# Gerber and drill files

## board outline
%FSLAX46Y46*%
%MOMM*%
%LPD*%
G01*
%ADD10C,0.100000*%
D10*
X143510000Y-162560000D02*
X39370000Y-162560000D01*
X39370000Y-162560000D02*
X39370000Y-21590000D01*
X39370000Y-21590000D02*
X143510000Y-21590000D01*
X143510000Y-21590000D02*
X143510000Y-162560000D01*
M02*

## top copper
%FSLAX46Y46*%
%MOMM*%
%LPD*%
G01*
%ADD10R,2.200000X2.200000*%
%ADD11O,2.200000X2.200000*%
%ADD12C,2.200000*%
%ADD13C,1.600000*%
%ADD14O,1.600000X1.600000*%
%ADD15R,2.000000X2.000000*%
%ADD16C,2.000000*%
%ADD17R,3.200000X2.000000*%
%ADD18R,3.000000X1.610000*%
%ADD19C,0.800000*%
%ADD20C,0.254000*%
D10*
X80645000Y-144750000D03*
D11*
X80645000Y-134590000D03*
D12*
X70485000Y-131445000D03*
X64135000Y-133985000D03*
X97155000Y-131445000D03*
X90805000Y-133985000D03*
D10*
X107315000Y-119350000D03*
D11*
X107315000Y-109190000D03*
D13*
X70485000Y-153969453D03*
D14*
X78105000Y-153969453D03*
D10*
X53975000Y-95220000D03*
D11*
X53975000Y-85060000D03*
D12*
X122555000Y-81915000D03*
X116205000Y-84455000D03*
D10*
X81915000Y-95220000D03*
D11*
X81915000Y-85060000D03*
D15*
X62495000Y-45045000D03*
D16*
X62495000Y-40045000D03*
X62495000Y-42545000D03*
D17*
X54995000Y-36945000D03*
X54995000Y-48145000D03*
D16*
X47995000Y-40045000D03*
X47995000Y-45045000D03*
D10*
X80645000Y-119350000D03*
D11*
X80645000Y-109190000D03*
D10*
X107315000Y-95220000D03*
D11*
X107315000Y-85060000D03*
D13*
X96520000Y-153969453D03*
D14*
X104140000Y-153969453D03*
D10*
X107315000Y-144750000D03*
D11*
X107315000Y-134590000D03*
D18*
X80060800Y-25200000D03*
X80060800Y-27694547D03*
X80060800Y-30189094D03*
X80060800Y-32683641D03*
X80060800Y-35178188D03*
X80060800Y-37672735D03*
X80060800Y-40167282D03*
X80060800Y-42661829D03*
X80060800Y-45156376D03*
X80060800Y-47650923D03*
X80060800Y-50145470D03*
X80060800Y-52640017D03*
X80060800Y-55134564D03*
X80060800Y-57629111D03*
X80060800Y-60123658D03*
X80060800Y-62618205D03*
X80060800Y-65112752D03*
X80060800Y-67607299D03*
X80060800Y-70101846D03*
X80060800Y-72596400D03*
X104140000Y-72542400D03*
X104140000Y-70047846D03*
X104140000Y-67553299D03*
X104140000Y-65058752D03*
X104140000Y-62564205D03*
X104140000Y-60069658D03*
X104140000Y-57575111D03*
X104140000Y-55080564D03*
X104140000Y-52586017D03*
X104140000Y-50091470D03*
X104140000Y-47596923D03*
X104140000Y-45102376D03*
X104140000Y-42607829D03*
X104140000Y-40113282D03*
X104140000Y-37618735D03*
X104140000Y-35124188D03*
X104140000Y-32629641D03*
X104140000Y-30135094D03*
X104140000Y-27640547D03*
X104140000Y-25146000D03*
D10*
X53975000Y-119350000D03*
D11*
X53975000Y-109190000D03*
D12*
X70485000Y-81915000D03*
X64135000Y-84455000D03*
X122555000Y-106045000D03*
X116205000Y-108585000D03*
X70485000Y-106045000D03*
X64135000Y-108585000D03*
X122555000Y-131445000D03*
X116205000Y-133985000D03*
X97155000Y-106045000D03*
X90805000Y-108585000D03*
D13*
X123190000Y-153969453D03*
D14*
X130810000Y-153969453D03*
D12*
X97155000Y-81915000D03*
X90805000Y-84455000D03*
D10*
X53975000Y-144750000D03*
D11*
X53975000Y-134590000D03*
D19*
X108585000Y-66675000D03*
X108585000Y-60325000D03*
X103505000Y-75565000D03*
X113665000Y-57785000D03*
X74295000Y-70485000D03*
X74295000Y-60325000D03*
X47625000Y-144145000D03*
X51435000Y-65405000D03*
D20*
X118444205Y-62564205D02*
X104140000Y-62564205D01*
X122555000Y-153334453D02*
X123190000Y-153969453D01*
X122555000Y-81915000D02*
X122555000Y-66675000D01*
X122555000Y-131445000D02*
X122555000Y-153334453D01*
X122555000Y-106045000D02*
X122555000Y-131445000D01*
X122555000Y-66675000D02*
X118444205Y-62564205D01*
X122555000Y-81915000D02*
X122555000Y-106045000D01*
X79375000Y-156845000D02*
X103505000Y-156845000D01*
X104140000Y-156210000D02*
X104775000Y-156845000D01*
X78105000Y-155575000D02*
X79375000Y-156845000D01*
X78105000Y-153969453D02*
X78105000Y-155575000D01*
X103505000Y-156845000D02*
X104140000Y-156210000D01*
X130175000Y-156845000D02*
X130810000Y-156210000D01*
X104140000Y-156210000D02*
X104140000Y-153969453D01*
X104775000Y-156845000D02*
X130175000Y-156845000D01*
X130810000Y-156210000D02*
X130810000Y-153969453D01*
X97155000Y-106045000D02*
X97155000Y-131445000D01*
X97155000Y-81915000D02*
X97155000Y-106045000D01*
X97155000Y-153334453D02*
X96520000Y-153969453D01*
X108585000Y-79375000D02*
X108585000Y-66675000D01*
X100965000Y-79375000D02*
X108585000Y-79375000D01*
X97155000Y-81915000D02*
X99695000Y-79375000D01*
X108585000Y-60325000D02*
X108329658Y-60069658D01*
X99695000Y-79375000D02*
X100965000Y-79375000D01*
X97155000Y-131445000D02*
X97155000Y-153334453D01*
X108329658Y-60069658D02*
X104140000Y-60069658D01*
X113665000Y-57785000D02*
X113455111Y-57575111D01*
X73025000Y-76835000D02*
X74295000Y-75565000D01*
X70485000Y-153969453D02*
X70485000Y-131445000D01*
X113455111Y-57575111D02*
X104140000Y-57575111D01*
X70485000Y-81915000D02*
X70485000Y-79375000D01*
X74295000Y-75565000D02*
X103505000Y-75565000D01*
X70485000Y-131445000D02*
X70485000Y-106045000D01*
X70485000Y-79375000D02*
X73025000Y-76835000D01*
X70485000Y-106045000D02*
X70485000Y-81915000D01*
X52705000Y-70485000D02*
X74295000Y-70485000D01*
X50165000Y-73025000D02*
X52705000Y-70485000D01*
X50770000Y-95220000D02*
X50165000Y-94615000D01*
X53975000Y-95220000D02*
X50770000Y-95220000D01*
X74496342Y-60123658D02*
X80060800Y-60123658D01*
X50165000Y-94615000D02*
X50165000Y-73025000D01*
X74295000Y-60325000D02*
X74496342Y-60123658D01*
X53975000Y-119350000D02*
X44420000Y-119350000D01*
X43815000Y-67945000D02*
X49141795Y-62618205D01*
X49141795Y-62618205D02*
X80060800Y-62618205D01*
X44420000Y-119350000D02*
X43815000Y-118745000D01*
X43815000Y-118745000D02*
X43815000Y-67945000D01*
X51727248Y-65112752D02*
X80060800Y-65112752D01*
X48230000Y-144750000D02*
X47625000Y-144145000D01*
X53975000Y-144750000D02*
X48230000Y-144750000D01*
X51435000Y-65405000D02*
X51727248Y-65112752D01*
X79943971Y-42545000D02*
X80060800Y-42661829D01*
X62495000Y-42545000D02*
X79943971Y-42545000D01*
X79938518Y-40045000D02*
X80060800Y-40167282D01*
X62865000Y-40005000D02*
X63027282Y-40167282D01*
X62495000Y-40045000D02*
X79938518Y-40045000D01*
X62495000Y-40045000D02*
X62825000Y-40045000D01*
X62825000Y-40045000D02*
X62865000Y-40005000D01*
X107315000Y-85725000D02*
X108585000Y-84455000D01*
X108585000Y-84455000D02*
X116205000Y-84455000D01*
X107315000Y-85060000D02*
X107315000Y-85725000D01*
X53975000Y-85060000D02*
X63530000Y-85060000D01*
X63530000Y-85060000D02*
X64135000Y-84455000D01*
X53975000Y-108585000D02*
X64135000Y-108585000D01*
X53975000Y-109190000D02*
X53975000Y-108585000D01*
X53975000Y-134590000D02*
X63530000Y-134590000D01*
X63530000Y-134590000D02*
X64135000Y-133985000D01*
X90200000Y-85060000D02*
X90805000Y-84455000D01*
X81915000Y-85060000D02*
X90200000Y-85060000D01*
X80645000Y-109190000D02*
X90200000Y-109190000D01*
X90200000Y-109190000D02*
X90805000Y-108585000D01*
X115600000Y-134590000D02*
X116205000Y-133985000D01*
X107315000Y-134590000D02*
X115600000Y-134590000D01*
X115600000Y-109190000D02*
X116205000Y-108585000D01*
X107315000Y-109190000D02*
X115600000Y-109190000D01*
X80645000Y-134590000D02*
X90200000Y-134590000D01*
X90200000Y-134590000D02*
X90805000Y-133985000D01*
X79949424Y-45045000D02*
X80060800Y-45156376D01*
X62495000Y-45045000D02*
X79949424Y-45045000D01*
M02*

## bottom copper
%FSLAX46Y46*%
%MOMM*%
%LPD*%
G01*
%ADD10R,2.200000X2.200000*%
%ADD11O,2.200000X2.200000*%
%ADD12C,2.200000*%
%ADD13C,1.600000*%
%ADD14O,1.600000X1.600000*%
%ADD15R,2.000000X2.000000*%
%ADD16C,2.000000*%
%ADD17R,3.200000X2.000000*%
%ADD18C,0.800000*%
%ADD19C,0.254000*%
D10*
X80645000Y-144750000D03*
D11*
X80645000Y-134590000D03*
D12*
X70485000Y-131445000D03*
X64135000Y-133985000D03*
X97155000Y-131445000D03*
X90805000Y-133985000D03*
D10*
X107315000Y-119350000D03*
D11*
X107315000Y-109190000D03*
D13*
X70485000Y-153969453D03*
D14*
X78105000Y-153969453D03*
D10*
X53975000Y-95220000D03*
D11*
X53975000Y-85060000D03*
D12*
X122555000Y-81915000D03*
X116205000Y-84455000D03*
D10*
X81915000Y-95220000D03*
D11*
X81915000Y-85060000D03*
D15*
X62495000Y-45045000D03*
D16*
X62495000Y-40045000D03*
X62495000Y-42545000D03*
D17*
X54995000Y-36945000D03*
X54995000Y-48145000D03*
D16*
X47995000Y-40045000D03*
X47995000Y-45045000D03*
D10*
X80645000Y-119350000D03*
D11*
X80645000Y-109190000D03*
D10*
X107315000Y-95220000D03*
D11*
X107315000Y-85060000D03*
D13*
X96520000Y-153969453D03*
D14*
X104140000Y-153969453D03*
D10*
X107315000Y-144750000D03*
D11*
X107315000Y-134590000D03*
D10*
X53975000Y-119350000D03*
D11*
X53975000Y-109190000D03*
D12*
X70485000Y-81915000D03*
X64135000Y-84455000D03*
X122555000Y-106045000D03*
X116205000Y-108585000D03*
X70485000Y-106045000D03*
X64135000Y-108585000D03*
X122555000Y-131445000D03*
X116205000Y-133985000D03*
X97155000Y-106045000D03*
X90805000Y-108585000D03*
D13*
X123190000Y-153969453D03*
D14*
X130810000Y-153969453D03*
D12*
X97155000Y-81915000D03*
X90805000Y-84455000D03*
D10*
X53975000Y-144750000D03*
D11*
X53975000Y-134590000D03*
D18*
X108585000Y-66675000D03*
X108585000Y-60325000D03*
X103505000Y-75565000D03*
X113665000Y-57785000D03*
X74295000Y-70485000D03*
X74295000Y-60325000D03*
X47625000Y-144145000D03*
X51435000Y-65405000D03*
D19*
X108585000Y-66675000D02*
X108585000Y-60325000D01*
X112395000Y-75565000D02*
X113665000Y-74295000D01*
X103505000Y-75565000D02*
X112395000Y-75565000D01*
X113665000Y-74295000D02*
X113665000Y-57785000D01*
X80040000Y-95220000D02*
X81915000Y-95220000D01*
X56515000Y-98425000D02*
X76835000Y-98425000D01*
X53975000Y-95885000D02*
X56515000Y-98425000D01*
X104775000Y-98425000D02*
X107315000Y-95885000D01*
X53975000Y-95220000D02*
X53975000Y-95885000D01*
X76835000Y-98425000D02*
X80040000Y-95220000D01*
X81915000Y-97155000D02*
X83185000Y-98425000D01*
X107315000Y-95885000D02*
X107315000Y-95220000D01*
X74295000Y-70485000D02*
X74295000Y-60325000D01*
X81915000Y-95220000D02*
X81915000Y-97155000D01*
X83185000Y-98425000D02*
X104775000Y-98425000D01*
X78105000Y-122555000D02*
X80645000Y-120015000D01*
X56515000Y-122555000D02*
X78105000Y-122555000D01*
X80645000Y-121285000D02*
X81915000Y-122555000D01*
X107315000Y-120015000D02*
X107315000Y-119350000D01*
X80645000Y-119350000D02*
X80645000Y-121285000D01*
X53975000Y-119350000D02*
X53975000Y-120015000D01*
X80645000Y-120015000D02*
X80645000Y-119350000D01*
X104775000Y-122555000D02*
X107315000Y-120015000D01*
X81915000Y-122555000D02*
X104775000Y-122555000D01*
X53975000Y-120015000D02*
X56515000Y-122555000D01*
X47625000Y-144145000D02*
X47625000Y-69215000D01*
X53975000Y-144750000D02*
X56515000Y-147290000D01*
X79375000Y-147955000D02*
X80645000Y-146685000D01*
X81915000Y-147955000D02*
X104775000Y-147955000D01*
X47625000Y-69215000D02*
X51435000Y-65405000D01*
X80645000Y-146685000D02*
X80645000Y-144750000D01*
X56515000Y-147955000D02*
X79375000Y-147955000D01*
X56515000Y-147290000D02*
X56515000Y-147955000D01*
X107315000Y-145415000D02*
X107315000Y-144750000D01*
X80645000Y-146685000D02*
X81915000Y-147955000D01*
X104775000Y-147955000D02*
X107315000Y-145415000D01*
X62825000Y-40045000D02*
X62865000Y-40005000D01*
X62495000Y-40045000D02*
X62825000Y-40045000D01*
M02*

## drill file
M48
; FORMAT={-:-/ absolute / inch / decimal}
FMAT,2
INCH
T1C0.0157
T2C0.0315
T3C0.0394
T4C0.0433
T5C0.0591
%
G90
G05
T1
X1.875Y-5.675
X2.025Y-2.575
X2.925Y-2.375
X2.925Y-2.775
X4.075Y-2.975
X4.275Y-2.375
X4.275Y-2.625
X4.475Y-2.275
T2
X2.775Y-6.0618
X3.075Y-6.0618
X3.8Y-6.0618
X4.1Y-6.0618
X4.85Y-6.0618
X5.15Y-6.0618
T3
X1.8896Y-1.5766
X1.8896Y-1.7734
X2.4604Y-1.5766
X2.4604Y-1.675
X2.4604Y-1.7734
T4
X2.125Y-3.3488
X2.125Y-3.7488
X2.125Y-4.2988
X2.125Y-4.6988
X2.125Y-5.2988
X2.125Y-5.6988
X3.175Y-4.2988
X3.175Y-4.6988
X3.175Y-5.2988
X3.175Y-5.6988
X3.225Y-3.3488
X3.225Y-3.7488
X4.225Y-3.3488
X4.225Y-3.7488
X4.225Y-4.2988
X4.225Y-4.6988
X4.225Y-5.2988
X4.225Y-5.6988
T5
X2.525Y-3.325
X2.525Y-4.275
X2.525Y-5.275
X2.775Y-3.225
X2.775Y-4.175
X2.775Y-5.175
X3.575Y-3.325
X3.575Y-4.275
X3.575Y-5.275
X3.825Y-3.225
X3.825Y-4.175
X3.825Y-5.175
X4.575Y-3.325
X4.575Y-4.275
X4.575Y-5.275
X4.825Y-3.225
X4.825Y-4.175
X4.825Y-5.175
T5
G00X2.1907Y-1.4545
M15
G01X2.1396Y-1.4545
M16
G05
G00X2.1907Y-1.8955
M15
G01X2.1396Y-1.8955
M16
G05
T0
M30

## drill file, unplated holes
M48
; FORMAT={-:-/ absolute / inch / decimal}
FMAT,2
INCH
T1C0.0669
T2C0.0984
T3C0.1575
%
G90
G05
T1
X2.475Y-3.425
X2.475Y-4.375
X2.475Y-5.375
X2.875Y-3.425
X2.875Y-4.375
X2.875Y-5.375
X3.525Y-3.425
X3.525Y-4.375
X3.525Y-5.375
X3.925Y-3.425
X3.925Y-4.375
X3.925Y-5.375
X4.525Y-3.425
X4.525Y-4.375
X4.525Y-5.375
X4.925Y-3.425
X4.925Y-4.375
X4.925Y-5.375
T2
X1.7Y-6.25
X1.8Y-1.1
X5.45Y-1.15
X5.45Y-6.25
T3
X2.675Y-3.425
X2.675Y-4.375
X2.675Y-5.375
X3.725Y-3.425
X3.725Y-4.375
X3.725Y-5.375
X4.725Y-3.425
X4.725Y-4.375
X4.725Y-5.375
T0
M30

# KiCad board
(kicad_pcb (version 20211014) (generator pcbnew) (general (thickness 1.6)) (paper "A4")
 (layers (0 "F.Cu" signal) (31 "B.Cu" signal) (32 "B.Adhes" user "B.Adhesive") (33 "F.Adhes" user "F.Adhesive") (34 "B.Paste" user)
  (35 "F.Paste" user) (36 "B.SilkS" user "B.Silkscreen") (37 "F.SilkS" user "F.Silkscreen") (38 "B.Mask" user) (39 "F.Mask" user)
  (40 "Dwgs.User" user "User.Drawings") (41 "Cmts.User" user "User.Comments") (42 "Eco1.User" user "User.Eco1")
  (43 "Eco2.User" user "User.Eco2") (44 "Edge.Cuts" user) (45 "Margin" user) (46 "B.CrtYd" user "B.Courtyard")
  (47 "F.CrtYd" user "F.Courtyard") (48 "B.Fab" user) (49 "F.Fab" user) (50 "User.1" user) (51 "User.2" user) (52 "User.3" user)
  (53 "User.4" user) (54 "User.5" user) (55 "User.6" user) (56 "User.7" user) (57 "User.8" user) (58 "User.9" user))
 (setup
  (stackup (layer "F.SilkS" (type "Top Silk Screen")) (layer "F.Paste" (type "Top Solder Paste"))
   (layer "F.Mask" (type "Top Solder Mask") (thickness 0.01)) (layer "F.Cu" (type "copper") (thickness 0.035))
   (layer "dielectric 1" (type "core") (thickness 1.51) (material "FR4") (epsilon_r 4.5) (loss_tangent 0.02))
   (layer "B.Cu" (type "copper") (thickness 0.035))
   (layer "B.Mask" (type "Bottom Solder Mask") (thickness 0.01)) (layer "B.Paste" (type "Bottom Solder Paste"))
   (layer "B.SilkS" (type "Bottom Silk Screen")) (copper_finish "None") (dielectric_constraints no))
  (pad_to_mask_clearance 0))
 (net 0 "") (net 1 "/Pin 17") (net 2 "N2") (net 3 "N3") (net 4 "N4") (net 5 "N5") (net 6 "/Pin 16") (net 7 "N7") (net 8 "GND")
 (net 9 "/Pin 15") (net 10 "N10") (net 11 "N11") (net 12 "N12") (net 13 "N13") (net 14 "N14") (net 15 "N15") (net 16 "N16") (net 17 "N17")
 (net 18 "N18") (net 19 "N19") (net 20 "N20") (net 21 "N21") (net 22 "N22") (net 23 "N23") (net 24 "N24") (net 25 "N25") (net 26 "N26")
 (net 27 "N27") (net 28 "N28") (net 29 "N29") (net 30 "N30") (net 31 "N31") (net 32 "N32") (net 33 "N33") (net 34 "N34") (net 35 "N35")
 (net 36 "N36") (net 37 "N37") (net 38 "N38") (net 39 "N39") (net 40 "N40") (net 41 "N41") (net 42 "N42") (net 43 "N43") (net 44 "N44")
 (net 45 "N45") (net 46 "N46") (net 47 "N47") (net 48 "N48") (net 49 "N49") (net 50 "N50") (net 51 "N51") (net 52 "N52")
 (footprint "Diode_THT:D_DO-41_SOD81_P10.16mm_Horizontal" (layer "F.Cu") (at 80.645 144.75 90)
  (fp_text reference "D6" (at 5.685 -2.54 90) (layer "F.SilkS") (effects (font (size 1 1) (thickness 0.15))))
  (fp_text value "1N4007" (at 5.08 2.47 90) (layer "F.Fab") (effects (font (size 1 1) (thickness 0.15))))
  (pad "1" thru_hole rect (at 0 0 90) (size 2.2 2.2) (drill 1.1) (layers *.Cu *.Mask) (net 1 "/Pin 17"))
  (pad "2" thru_hole oval (at 10.16 0 90) (size 2.2 2.2) (drill 1.1) (layers *.Cu *.Mask) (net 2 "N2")))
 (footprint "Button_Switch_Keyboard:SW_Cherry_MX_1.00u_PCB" (layer "F.Cu") (at 70.485 131.445)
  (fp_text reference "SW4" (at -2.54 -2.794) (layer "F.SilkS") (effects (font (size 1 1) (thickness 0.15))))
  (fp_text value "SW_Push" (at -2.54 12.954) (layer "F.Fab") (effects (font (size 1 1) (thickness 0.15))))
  (pad "" np_thru_hole circle (at -7.62 5.08) (size 1.7 1.7) (drill 1.7) (layers *.Cu *.Mask))
  (pad "" np_thru_hole circle (at -2.54 5.08) (size 4 4) (drill 4) (layers *.Cu *.Mask))
  (pad "" np_thru_hole circle (at 2.54 5.08) (size 1.7 1.7) (drill 1.7) (layers *.Cu *.Mask))
  (pad "1" thru_hole circle (at 0 0) (size 2.2 2.2) (drill 1.5) (layers *.Cu *.Mask) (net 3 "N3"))
  (pad "2" thru_hole circle (at -6.35 2.54) (size 2.2 2.2) (drill 1.5) (layers *.Cu *.Mask) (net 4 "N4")))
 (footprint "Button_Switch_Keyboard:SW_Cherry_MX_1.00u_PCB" (layer "F.Cu") (at 97.155 131.445)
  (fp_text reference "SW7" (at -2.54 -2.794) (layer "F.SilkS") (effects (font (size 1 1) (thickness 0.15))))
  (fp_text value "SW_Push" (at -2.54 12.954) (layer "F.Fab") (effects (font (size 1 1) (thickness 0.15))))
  (pad "" np_thru_hole circle (at -7.62 5.08) (size 1.7 1.7) (drill 1.7) (layers *.Cu *.Mask))
  (pad "" np_thru_hole circle (at 2.54 5.08) (size 1.7 1.7) (drill 1.7) (layers *.Cu *.Mask))
  (pad "" np_thru_hole circle (at -2.54 5.08) (size 4 4) (drill 4) (layers *.Cu *.Mask))
  (pad "1" thru_hole circle (at 0 0) (size 2.2 2.2) (drill 1.5) (layers *.Cu *.Mask) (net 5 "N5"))
  (pad "2" thru_hole circle (at -6.35 2.54) (size 2.2 2.2) (drill 1.5) (layers *.Cu *.Mask) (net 2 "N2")))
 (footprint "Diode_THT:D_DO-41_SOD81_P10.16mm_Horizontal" (layer "F.Cu") (at 107.315 119.35 90)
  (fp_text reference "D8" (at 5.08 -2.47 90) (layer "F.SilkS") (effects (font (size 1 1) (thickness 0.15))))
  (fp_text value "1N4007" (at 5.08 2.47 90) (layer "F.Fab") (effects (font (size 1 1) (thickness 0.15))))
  (pad "1" thru_hole rect (at 0 0 90) (size 2.2 2.2) (drill 1.1) (layers *.Cu *.Mask) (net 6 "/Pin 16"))
  (pad "2" thru_hole oval (at 10.16 0 90) (size 2.2 2.2) (drill 1.1) (layers *.Cu *.Mask) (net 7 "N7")))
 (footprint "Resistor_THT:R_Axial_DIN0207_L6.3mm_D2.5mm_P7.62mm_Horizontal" (layer "F.Cu") (at 70.485 153.969453)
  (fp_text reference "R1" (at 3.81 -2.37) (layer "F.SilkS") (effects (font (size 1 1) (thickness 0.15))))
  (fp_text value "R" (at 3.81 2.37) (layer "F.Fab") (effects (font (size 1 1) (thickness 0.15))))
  (pad "1" thru_hole circle (at 0 0) (size 1.6 1.6) (drill 0.8) (layers *.Cu *.Mask) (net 3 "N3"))
  (pad "2" thru_hole oval (at 7.62 0) (size 1.6 1.6) (drill 0.8) (layers *.Cu *.Mask) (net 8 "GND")))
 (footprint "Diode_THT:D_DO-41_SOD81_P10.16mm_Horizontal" (layer "F.Cu") (at 53.975 95.22 90)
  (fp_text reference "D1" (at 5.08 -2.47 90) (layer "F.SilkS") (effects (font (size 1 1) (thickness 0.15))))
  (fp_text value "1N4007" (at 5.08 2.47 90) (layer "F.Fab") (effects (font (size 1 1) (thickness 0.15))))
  (pad "1" thru_hole rect (at 0 0 90) (size 2.2 2.2) (drill 1.1) (layers *.Cu *.Mask) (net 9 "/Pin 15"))
  (pad "2" thru_hole oval (at 10.16 0 90) (size 2.2 2.2) (drill 1.1) (layers *.Cu *.Mask) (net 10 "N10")))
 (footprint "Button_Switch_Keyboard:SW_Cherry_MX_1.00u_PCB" (layer "F.Cu") (at 122.555 81.915)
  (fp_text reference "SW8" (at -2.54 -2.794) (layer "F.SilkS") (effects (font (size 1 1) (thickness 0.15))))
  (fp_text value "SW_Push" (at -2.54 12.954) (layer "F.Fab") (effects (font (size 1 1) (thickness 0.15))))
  (pad "" np_thru_hole circle (at 2.54 5.08) (size 1.7 1.7) (drill 1.7) (layers *.Cu *.Mask))
  (pad "" np_thru_hole circle (at -2.54 5.08) (size 4 4) (drill 4) (layers *.Cu *.Mask))
  (pad "" np_thru_hole circle (at -7.62 5.08) (size 1.7 1.7) (drill 1.7) (layers *.Cu *.Mask))
  (pad "1" thru_hole circle (at 0 0) (size 2.2 2.2) (drill 1.5) (layers *.Cu *.Mask) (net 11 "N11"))
  (pad "2" thru_hole circle (at -6.35 2.54) (size 2.2 2.2) (drill 1.5) (layers *.Cu *.Mask) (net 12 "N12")))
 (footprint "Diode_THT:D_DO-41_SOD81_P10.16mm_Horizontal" (layer "F.Cu") (at 81.915 95.22 90)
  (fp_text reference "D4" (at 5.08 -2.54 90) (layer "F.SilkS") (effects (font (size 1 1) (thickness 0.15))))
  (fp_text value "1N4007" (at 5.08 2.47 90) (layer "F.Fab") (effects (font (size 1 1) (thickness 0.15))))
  (pad "1" thru_hole rect (at 0 0 90) (size 2.2 2.2) (drill 1.1) (layers *.Cu *.Mask) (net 9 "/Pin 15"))
  (pad "2" thru_hole oval (at 10.16 0 90) (size 2.2 2.2) (drill 1.1) (layers *.Cu *.Mask) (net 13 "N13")))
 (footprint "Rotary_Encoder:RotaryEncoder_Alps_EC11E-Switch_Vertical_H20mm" (layer "F.Cu") (at 62.495 45.045 180)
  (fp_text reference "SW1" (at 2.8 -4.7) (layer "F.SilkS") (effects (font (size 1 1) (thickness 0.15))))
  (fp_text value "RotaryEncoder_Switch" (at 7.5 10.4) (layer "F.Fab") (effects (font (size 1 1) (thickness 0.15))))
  (pad "A" thru_hole rect (at 0 0 180) (size 2 2) (drill 1) (layers *.Cu *.Mask) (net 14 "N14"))
  (pad "B" thru_hole circle (at 0 5 180) (size 2 2) (drill 1) (layers *.Cu *.Mask) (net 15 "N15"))
  (pad "C" thru_hole circle (at 0 2.5 180) (size 2 2) (drill 1) (layers *.Cu *.Mask) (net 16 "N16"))
  (pad "MP" thru_hole rect (at 7.5 8.1 180) (size 3.2 2) (drill oval 2.8 1.5) (layers *.Cu *.Mask))
  (pad "MP" thru_hole rect (at 7.5 -3.1 180) (size 3.2 2) (drill oval 2.8 1.5) (layers *.Cu *.Mask))
  (pad "S1" thru_hole circle (at 14.5 5 180) (size 2 2) (drill 1) (layers *.Cu *.Mask) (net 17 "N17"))
  (pad "S2" thru_hole circle (at 14.5 0 180) (size 2 2) (drill 1) (layers *.Cu *.Mask) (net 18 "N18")))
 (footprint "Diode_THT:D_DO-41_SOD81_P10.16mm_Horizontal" (layer "F.Cu") (at 80.645 119.35 90)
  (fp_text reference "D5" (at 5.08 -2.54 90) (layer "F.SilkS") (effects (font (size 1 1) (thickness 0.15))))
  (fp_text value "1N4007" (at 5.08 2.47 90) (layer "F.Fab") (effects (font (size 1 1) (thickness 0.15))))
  (pad "1" thru_hole rect (at 0 0 90) (size 2.2 2.2) (drill 1.1) (layers *.Cu *.Mask) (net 6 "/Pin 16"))
  (pad "2" thru_hole oval (at 10.16 0 90) (size 2.2 2.2) (drill 1.1) (layers *.Cu *.Mask) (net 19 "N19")))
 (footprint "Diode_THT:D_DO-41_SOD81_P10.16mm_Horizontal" (layer "F.Cu") (at 107.315 95.22 90)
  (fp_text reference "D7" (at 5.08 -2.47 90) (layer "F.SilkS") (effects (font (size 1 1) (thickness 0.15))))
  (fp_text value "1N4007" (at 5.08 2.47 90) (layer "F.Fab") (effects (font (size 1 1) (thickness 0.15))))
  (pad "1" thru_hole rect (at 0 0 90) (size 2.2 2.2) (drill 1.1) (layers *.Cu *.Mask) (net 9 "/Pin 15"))
  (pad "2" thru_hole oval (at 10.16 0 90) (size 2.2 2.2) (drill 1.1) (layers *.Cu *.Mask) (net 12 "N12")))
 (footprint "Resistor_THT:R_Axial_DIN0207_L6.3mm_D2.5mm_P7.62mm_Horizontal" (layer "F.Cu") (at 96.52 153.969453)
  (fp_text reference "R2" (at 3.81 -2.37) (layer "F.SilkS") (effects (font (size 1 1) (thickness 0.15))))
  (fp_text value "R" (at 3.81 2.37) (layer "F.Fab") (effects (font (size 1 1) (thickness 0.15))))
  (pad "1" thru_hole circle (at 0 0) (size 1.6 1.6) (drill 0.8) (layers *.Cu *.Mask) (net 5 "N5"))
  (pad "2" thru_hole oval (at 7.62 0) (size 1.6 1.6) (drill 0.8) (layers *.Cu *.Mask) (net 8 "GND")))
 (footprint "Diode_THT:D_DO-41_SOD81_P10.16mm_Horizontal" (layer "F.Cu") (at 107.315 144.75 90)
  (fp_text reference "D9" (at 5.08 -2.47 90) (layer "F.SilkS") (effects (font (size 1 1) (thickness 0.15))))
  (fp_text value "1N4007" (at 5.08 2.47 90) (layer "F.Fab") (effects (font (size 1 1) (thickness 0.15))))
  (pad "1" thru_hole rect (at 0 0 90) (size 2.2 2.2) (drill 1.1) (layers *.Cu *.Mask) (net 1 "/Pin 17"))
  (pad "2" thru_hole oval (at 10.16 0 90) (size 2.2 2.2) (drill 1.1) (layers *.Cu *.Mask) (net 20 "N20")))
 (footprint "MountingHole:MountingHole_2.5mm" (layer "F.Cu") (at 138.43 158.75)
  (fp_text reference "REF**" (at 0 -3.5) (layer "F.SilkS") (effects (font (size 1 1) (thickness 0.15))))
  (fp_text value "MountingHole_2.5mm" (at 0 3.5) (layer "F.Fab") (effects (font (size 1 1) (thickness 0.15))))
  (pad "" np_thru_hole circle (at 0 0) (size 2.5 2.5) (drill 2.5) (layers *.Cu *.Mask)))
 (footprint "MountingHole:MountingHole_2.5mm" (layer "F.Cu") (at 43.18 158.75)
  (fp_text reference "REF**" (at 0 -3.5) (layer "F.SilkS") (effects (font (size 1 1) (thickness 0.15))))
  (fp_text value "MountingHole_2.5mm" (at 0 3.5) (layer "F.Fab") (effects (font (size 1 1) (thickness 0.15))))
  (pad "" np_thru_hole circle (at 0 0) (size 2.5 2.5) (drill 2.5) (layers *.Cu *.Mask)))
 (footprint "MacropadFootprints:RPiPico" (layer "F.Cu") (at 92.075 48.895)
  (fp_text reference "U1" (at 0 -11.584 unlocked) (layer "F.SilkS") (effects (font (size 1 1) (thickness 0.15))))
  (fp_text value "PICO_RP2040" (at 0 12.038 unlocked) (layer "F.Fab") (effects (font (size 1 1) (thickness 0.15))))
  (pad "1" smd rect (at -12.0142 -23.695) (size 3 1.61) (layers "F.Cu" "F.Paste" "F.Mask") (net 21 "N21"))
  (pad "2" smd rect (at -12.0142 -21.200453) (size 3 1.61) (layers "F.Cu" "F.Paste" "F.Mask") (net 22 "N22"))
  (pad "3" smd rect (at -12.0142 -18.705906) (size 3 1.61) (layers "F.Cu" "F.Paste" "F.Mask") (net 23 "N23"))
  (pad "4" smd rect (at -12.0142 -16.211359) (size 3 1.61) (layers "F.Cu" "F.Paste" "F.Mask") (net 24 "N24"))
  (pad "5" smd rect (at -12.0142 -13.716812) (size 3 1.61) (layers "F.Cu" "F.Paste" "F.Mask") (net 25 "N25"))
  (pad "6" smd rect (at -12.0142 -11.222265) (size 3 1.61) (layers "F.Cu" "F.Paste" "F.Mask") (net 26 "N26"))
  (pad "7" smd rect (at -12.0142 -8.727718) (size 3 1.61) (layers "F.Cu" "F.Paste" "F.Mask") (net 15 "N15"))
  (pad "8" smd rect (at -12.0142 -6.233171) (size 3 1.61) (layers "F.Cu" "F.Paste" "F.Mask") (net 16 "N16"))
  (pad "9" smd rect (at -12.0142 -3.738624) (size 3 1.61) (layers "F.Cu" "F.Paste" "F.Mask") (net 14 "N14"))
  (pad "10" smd rect (at -12.0142 -1.244077) (size 3 1.61) (layers "F.Cu" "F.Paste" "F.Mask") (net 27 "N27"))
  (pad "11" smd rect (at -12.0142 1.25047) (size 3 1.61) (layers "F.Cu" "F.Paste" "F.Mask") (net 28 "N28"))
  (pad "12" smd rect (at -12.0142 3.745017) (size 3 1.61) (layers "F.Cu" "F.Paste" "F.Mask") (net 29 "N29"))
  (pad "13" smd rect (at -12.0142 6.239564) (size 3 1.61) (layers "F.Cu" "F.Paste" "F.Mask") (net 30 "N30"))
  (pad "14" smd rect (at -12.0142 8.734111) (size 3 1.61) (layers "F.Cu" "F.Paste" "F.Mask") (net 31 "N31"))
  (pad "15" smd rect (at -12.0142 11.228658) (size 3 1.61) (layers "F.Cu" "F.Paste" "F.Mask") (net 9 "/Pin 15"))
  (pad "16" smd rect (at -12.0142 13.723205) (size 3 1.61) (layers "F.Cu" "F.Paste" "F.Mask") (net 6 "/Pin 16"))
  (pad "17" smd rect (at -12.0142 16.217752) (size 3 1.61) (layers "F.Cu" "F.Paste" "F.Mask") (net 1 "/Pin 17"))
  (pad "18" smd rect (at -12.0142 18.712299) (size 3 1.61) (layers "F.Cu" "F.Paste" "F.Mask") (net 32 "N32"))
  (pad "19" smd rect (at -12.0142 21.206846) (size 3 1.61) (layers "F.Cu" "F.Paste" "F.Mask") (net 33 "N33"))
  (pad "20" smd rect (at -12.0142 23.7014) (size 3 1.61) (layers "F.Cu" "F.Paste" "F.Mask") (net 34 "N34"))
  (pad "21" smd rect (at 12.065 23.6474) (size 3 1.61) (layers "F.Cu" "F.Paste" "F.Mask") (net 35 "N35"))
  (pad "22" smd rect (at 12.065 21.152846) (size 3 1.61) (layers "F.Cu" "F.Paste" "F.Mask") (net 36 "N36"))
  (pad "23" smd rect (at 12.065 18.658299) (size 3 1.61) (layers "F.Cu" "F.Paste" "F.Mask") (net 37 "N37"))
  (pad "24" smd rect (at 12.065 16.163752) (size 3 1.61) (layers "F.Cu" "F.Paste" "F.Mask") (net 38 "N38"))
  (pad "25" smd rect (at 12.065 13.669205) (size 3 1.61) (layers "F.Cu" "F.Paste" "F.Mask") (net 11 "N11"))
  (pad "26" smd rect (at 12.065 11.174658) (size 3 1.61) (layers "F.Cu" "F.Paste" "F.Mask") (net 5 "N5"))
  (pad "27" smd rect (at 12.065 8.680111) (size 3 1.61) (layers "F.Cu" "F.Paste" "F.Mask") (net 3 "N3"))
  (pad "28" smd rect (at 12.065 6.185564) (size 3 1.61) (layers "F.Cu" "F.Paste" "F.Mask") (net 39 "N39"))
  (pad "29" smd rect (at 12.065 3.691017) (size 3 1.61) (layers "F.Cu" "F.Paste" "F.Mask") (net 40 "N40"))
  (pad "30" smd rect (at 12.065 1.19647) (size 3 1.61) (layers "F.Cu" "F.Paste" "F.Mask") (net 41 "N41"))
  (pad "31" smd rect (at 12.065 -1.298077) (size 3 1.61) (layers "F.Cu" "F.Paste" "F.Mask") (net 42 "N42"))
  (pad "32" smd rect (at 12.065 -3.792624) (size 3 1.61) (layers "F.Cu" "F.Paste" "F.Mask") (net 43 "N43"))
  (pad "33" smd rect (at 12.065 -6.287171) (size 3 1.61) (layers "F.Cu" "F.Paste" "F.Mask") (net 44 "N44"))
  (pad "34" smd rect (at 12.065 -8.781718) (size 3 1.61) (layers "F.Cu" "F.Paste" "F.Mask") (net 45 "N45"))
  (pad "35" smd rect (at 12.065 -11.276265) (size 3 1.61) (layers "F.Cu" "F.Paste" "F.Mask") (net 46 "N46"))
  (pad "36" smd rect (at 12.065 -13.770812) (size 3 1.61) (layers "F.Cu" "F.Paste" "F.Mask") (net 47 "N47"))
  (pad "37" smd rect (at 12.065 -16.265359) (size 3 1.61) (layers "F.Cu" "F.Paste" "F.Mask") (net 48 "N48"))
  (pad "38" smd rect (at 12.065 -18.759906) (size 3 1.61) (layers "F.Cu" "F.Paste" "F.Mask") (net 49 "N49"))
  (pad "39" smd rect (at 12.065 -21.254453) (size 3 1.61) (layers "F.Cu" "F.Paste" "F.Mask") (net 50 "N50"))
  (pad "40" smd rect (at 12.065 -23.749) (size 3 1.61) (layers "F.Cu" "F.Paste" "F.Mask") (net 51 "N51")))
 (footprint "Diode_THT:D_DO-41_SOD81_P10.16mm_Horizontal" (layer "F.Cu") (at 53.975 119.35 90)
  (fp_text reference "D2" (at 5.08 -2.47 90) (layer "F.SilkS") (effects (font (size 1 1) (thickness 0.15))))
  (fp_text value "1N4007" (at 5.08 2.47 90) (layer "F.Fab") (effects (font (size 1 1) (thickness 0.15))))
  (pad "1" thru_hole rect (at 0 0 90) (size 2.2 2.2) (drill 1.1) (layers *.Cu *.Mask) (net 6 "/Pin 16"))
  (pad "2" thru_hole oval (at 10.16 0 90) (size 2.2 2.2) (drill 1.1) (layers *.Cu *.Mask) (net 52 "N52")))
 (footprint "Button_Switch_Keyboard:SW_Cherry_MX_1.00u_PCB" (layer "F.Cu") (at 70.485 81.915)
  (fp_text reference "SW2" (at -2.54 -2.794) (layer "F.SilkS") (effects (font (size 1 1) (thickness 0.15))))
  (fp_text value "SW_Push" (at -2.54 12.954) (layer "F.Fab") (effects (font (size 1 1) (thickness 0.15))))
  (pad "" np_thru_hole circle (at -7.62 5.08) (size 1.7 1.7) (drill 1.7) (layers *.Cu *.Mask))
  (pad "" np_thru_hole circle (at -2.54 5.08) (size 4 4) (drill 4) (layers *.Cu *.Mask))
  (pad "" np_thru_hole circle (at 2.54 5.08) (size 1.7 1.7) (drill 1.7) (layers *.Cu *.Mask))
  (pad "1" thru_hole circle (at 0 0) (size 2.2 2.2) (drill 1.5) (layers *.Cu *.Mask) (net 3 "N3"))
  (pad "2" thru_hole circle (at -6.35 2.54) (size 2.2 2.2) (drill 1.5) (layers *.Cu *.Mask) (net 10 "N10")))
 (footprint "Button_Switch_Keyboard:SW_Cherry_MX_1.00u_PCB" (layer "F.Cu") (at 122.555 106.045)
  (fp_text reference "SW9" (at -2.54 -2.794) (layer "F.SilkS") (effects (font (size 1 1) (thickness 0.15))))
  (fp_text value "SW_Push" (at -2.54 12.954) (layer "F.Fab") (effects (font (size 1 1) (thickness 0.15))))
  (pad "" np_thru_hole circle (at 2.54 5.08) (size 1.7 1.7) (drill 1.7) (layers *.Cu *.Mask))
  (pad "" np_thru_hole circle (at -7.62 5.08) (size 1.7 1.7) (drill 1.7) (layers *.Cu *.Mask))
  (pad "" np_thru_hole circle (at -2.54 5.08) (size 4 4) (drill 4) (layers *.Cu *.Mask))
  (pad "1" thru_hole circle (at 0 0) (size 2.2 2.2) (drill 1.5) (layers *.Cu *.Mask) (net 11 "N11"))
  (pad "2" thru_hole circle (at -6.35 2.54) (size 2.2 2.2) (drill 1.5) (layers *.Cu *.Mask) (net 7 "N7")))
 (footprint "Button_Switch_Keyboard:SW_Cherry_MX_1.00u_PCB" (layer "F.Cu") (at 70.485 106.045)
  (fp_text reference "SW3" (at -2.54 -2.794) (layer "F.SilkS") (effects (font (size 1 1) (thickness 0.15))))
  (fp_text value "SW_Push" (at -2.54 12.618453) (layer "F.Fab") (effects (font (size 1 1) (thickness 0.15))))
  (pad "" np_thru_hole circle (at 2.54 5.08) (size 1.7 1.7) (drill 1.7) (layers *.Cu *.Mask))
  (pad "" np_thru_hole circle (at -7.62 5.08) (size 1.7 1.7) (drill 1.7) (layers *.Cu *.Mask))
  (pad "" np_thru_hole circle (at -2.54 5.08) (size 4 4) (drill 4) (layers *.Cu *.Mask))
  (pad "1" thru_hole circle (at 0 0) (size 2.2 2.2) (drill 1.5) (layers *.Cu *.Mask) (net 3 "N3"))
  (pad "2" thru_hole circle (at -6.35 2.54) (size 2.2 2.2) (drill 1.5) (layers *.Cu *.Mask) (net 52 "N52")))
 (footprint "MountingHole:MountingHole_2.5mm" (layer "F.Cu") (at 45.72 27.94)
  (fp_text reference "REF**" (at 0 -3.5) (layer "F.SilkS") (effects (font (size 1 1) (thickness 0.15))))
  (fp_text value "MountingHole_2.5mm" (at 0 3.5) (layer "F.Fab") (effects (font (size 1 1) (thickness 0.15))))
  (pad "" np_thru_hole circle (at 0 0) (size 2.5 2.5) (drill 2.5) (layers *.Cu *.Mask)))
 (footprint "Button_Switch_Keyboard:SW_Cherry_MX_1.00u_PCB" (layer "F.Cu") (at 122.555 131.445)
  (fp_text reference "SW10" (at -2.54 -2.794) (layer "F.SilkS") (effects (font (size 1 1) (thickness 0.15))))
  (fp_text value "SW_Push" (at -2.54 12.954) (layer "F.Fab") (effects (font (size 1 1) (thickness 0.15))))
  (pad "" np_thru_hole circle (at -2.54 5.08) (size 4 4) (drill 4) (layers *.Cu *.Mask))
  (pad "" np_thru_hole circle (at 2.54 5.08) (size 1.7 1.7) (drill 1.7) (layers *.Cu *.Mask))
  (pad "" np_thru_hole circle (at -7.62 5.08) (size 1.7 1.7) (drill 1.7) (layers *.Cu *.Mask))
  (pad "1" thru_hole circle (at 0 0) (size 2.2 2.2) (drill 1.5) (layers *.Cu *.Mask) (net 11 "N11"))
  (pad "2" thru_hole circle (at -6.35 2.54) (size 2.2 2.2) (drill 1.5) (layers *.Cu *.Mask) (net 20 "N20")))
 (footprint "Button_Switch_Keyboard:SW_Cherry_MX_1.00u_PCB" (layer "F.Cu") (at 97.155 106.045)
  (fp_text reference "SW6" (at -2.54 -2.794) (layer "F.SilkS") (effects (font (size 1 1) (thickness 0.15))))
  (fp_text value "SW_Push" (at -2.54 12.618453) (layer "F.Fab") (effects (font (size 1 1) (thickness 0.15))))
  (pad "" np_thru_hole circle (at -7.62 5.08) (size 1.7 1.7) (drill 1.7) (layers *.Cu *.Mask))
  (pad "" np_thru_hole circle (at 2.54 5.08) (size 1.7 1.7) (drill 1.7) (layers *.Cu *.Mask))
  (pad "" np_thru_hole circle (at -2.54 5.08) (size 4 4) (drill 4) (layers *.Cu *.Mask))
  (pad "1" thru_hole circle (at 0 0) (size 2.2 2.2) (drill 1.5) (layers *.Cu *.Mask) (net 5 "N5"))
  (pad "2" thru_hole circle (at -6.35 2.54) (size 2.2 2.2) (drill 1.5) (layers *.Cu *.Mask) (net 19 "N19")))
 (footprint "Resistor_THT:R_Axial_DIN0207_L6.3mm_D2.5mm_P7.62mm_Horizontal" (layer "F.Cu") (at 123.19 153.969453)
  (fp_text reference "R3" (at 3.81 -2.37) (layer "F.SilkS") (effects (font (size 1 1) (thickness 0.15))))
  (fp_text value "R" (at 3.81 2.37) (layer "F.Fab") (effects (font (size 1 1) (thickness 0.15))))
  (pad "1" thru_hole circle (at 0 0) (size 1.6 1.6) (drill 0.8) (layers *.Cu *.Mask) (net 11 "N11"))
  (pad "2" thru_hole oval (at 7.62 0) (size 1.6 1.6) (drill 0.8) (layers *.Cu *.Mask) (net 8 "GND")))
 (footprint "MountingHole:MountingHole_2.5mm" (layer "F.Cu") (at 138.43 29.21)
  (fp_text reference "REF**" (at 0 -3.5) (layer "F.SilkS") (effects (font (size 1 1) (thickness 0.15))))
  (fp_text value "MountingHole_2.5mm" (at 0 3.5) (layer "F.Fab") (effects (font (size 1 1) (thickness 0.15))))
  (pad "" np_thru_hole circle (at 0 0) (size 2.5 2.5) (drill 2.5) (layers *.Cu *.Mask)))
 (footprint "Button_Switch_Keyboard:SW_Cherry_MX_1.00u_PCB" (layer "F.Cu") (at 97.155 81.915)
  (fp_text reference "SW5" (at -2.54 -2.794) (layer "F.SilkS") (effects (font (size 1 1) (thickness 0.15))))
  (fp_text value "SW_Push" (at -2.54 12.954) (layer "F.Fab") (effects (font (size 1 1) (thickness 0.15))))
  (pad "" np_thru_hole circle (at -2.54 5.08) (size 4 4) (drill 4) (layers *.Cu *.Mask))
  (pad "" np_thru_hole circle (at -7.62 5.08) (size 1.7 1.7) (drill 1.7) (layers *.Cu *.Mask))
  (pad "" np_thru_hole circle (at 2.54 5.08) (size 1.7 1.7) (drill 1.7) (layers *.Cu *.Mask))
  (pad "1" thru_hole circle (at 0 0) (size 2.2 2.2) (drill 1.5) (layers *.Cu *.Mask) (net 5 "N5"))
  (pad "2" thru_hole circle (at -6.35 2.54) (size 2.2 2.2) (drill 1.5) (layers *.Cu *.Mask) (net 13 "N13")))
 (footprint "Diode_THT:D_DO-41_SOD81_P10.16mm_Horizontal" (layer "F.Cu") (at 53.975 144.75 90)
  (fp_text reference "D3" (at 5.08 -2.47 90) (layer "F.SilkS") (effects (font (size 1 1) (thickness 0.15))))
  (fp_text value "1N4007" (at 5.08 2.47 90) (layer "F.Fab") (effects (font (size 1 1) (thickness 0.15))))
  (pad "1" thru_hole rect (at 0 0 90) (size 2.2 2.2) (drill 1.1) (layers *.Cu *.Mask) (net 1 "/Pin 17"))
  (pad "2" thru_hole oval (at 10.16 0 90) (size 2.2 2.2) (drill 1.1) (layers *.Cu *.Mask) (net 4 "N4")))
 (gr_rect (start 143.51 162.56) (end 39.37 21.59) (layer "Edge.Cuts") (width 0.1) (fill none))
 (segment (start 118.444205 62.564205) (end 104.14 62.564205) (width 0.254) (layer "F.Cu") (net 11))
 (segment (start 122.555 153.334453) (end 123.19 153.969453) (width 0.254) (layer "F.Cu") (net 11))
 (segment (start 122.555 81.915) (end 122.555 66.675) (width 0.254) (layer "F.Cu") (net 11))
 (segment (start 122.555 131.445) (end 122.555 153.334453) (width 0.254) (layer "F.Cu") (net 11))
 (segment (start 122.555 106.045) (end 122.555 131.445) (width 0.254) (layer "F.Cu") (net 11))
 (segment (start 122.555 66.675) (end 118.444205 62.564205) (width 0.254) (layer "F.Cu") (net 11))
 (segment (start 122.555 81.915) (end 122.555 106.045) (width 0.254) (layer "F.Cu") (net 11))
 (segment (start 79.375 156.845) (end 103.505 156.845) (width 0.254) (layer "F.Cu") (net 8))
 (segment (start 104.14 156.21) (end 104.775 156.845) (width 0.254) (layer "F.Cu") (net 8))
 (segment (start 78.105 155.575) (end 79.375 156.845) (width 0.254) (layer "F.Cu") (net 8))
 (segment (start 78.105 153.969453) (end 78.105 155.575) (width 0.254) (layer "F.Cu") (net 8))
 (segment (start 103.505 156.845) (end 104.14 156.21) (width 0.254) (layer "F.Cu") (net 8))
 (segment (start 130.175 156.845) (end 130.81 156.21) (width 0.254) (layer "F.Cu") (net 8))
 (segment (start 104.14 156.21) (end 104.14 153.969453) (width 0.254) (layer "F.Cu") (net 8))
 (segment (start 104.775 156.845) (end 130.175 156.845) (width 0.254) (layer "F.Cu") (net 8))
 (segment (start 130.81 156.21) (end 130.81 153.969453) (width 0.254) (layer "F.Cu") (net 8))
 (segment (start 97.155 106.045) (end 97.155 131.445) (width 0.254) (layer "F.Cu") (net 5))
 (segment (start 97.155 81.915) (end 97.155 106.045) (width 0.254) (layer "F.Cu") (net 5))
 (segment (start 97.155 153.334453) (end 96.52 153.969453) (width 0.254) (layer "F.Cu") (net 5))
 (segment (start 108.585 79.375) (end 108.585 66.675) (width 0.254) (layer "F.Cu") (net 5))
 (segment (start 100.965 79.375) (end 108.585 79.375) (width 0.254) (layer "F.Cu") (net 5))
 (segment (start 97.155 81.915) (end 99.695 79.375) (width 0.254) (layer "F.Cu") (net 5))
 (segment (start 108.585 60.325) (end 108.329658 60.069658) (width 0.254) (layer "F.Cu") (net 5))
 (segment (start 99.695 79.375) (end 100.965 79.375) (width 0.254) (layer "F.Cu") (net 5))
 (segment (start 97.155 131.445) (end 97.155 153.334453) (width 0.254) (layer "F.Cu") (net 5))
 (segment (start 108.329658 60.069658) (end 104.14 60.069658) (width 0.254) (layer "F.Cu") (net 5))
 (via (at 108.585 66.675) (size 0.8) (drill 0.4) (layers "F.Cu" "B.Cu") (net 5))
 (via (at 108.585 60.325) (size 0.8) (drill 0.4) (layers "F.Cu" "B.Cu") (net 5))
 (segment (start 108.585 66.675) (end 108.585 60.325) (width 0.254) (layer "B.Cu") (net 5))
 (segment (start 113.665 57.785) (end 113.455111 57.575111) (width 0.254) (layer "F.Cu") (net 3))
 (segment (start 73.025 76.835) (end 74.295 75.565) (width 0.254) (layer "F.Cu") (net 3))
 (segment (start 70.485 153.969453) (end 70.485 131.445) (width 0.254) (layer "F.Cu") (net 3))
 (segment (start 113.455111 57.575111) (end 104.14 57.575111) (width 0.254) (layer "F.Cu") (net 3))
 (segment (start 70.485 81.915) (end 70.485 79.375) (width 0.254) (layer "F.Cu") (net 3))
 (segment (start 74.295 75.565) (end 103.505 75.565) (width 0.254) (layer "F.Cu") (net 3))
 (segment (start 70.485 131.445) (end 70.485 106.045) (width 0.254) (layer "F.Cu") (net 3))
 (segment (start 70.485 79.375) (end 73.025 76.835) (width 0.254) (layer "F.Cu") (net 3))
 (segment (start 70.485 106.045) (end 70.485 81.915) (width 0.254) (layer "F.Cu") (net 3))
 (via (at 103.505 75.565) (size 0.8) (drill 0.4) (layers "F.Cu" "B.Cu") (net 3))
 (via (at 113.665 57.785) (size 0.8) (drill 0.4) (layers "F.Cu" "B.Cu") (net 3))
 (segment (start 112.395 75.565) (end 113.665 74.295) (width 0.254) (layer "B.Cu") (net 3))
 (segment (start 103.505 75.565) (end 112.395 75.565) (width 0.254) (layer "B.Cu") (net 3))
 (segment (start 113.665 74.295) (end 113.665 57.785) (width 0.254) (layer "B.Cu") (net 3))
 (segment (start 52.705 70.485) (end 74.295 70.485) (width 0.254) (layer "F.Cu") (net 9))
 (segment (start 50.165 73.025) (end 52.705 70.485) (width 0.254) (layer "F.Cu") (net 9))
 (segment (start 50.77 95.22) (end 50.165 94.615) (width 0.254) (layer "F.Cu") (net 9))
 (segment (start 53.975 95.22) (end 50.77 95.22) (width 0.254) (layer "F.Cu") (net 9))
 (segment (start 74.496342 60.123658) (end 80.0608 60.123658) (width 0.254) (layer "F.Cu") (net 9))
 (segment (start 50.165 94.615) (end 50.165 73.025) (width 0.254) (layer "F.Cu") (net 9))
 (segment (start 74.295 60.325) (end 74.496342 60.123658) (width 0.254) (layer "F.Cu") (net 9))
 (via (at 74.295 70.485) (size 0.8) (drill 0.4) (layers "F.Cu" "B.Cu") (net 9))
 (via (at 74.295 60.325) (size 0.8) (drill 0.4) (layers "F.Cu" "B.Cu") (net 9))
 (segment (start 80.04 95.22) (end 81.915 95.22) (width 0.254) (layer "B.Cu") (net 9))
 (segment (start 56.515 98.425) (end 76.835 98.425) (width 0.254) (layer "B.Cu") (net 9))
 (segment (start 53.975 95.885) (end 56.515 98.425) (width 0.254) (layer "B.Cu") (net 9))
 (segment (start 104.775 98.425) (end 107.315 95.885) (width 0.254) (layer "B.Cu") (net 9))
 (segment (start 53.975 95.22) (end 53.975 95.885) (width 0.254) (layer "B.Cu") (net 9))
 (segment (start 76.835 98.425) (end 80.04 95.22) (width 0.254) (layer "B.Cu") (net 9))
 (segment (start 81.915 97.155) (end 83.185 98.425) (width 0.254) (layer "B.Cu") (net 9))
 (segment (start 107.315 95.885) (end 107.315 95.22) (width 0.254) (layer "B.Cu") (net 9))
 (segment (start 74.295 70.485) (end 74.295 60.325) (width 0.254) (layer "B.Cu") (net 9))
 (segment (start 81.915 95.22) (end 81.915 97.155) (width 0.254) (layer "B.Cu") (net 9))
 (segment (start 83.185 98.425) (end 104.775 98.425) (width 0.254) (layer "B.Cu") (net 9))
 (segment (start 53.975 119.35) (end 44.42 119.35) (width 0.254) (layer "F.Cu") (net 6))
 (segment (start 43.815 67.945) (end 49.141795 62.618205) (width 0.254) (layer "F.Cu") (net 6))
 (segment (start 49.141795 62.618205) (end 80.0608 62.618205) (width 0.254) (layer "F.Cu") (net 6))
 (segment (start 44.42 119.35) (end 43.815 118.745) (width 0.254) (layer "F.Cu") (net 6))
 (segment (start 43.815 118.745) (end 43.815 67.945) (width 0.254) (layer "F.Cu") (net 6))
 (segment (start 78.105 122.555) (end 80.645 120.015) (width 0.254) (layer "B.Cu") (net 6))
 (segment (start 56.515 122.555) (end 78.105 122.555) (width 0.254) (layer "B.Cu") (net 6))
 (segment (start 80.645 121.285) (end 81.915 122.555) (width 0.254) (layer "B.Cu") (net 6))
 (segment (start 107.315 120.015) (end 107.315 119.35) (width 0.254) (layer "B.Cu") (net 6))
 (segment (start 80.645 119.35) (end 80.645 121.285) (width 0.254) (layer "B.Cu") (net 6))
 (segment (start 53.975 119.35) (end 53.975 120.015) (width 0.254) (layer "B.Cu") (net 6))
 (segment (start 80.645 120.015) (end 80.645 119.35) (width 0.254) (layer "B.Cu") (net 6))
 (segment (start 104.775 122.555) (end 107.315 120.015) (width 0.254) (layer "B.Cu") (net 6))
 (segment (start 81.915 122.555) (end 104.775 122.555) (width 0.254) (layer "B.Cu") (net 6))
 (segment (start 53.975 120.015) (end 56.515 122.555) (width 0.254) (layer "B.Cu") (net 6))
 (segment (start 51.727248 65.112752) (end 80.0608 65.112752) (width 0.254) (layer "F.Cu") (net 1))
 (segment (start 48.23 144.75) (end 47.625 144.145) (width 0.254) (layer "F.Cu") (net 1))
 (segment (start 53.975 144.75) (end 48.23 144.75) (width 0.254) (layer "F.Cu") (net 1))
 (segment (start 51.435 65.405) (end 51.727248 65.112752) (width 0.254) (layer "F.Cu") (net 1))
 (via (at 47.625 144.145) (size 0.8) (drill 0.4) (layers "F.Cu" "B.Cu") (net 1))
 (via (at 51.435 65.405) (size 0.8) (drill 0.4) (layers "F.Cu" "B.Cu") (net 1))
 (segment (start 47.625 144.145) (end 47.625 69.215) (width 0.254) (layer "B.Cu") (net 1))
 (segment (start 53.975 144.75) (end 56.515 147.29) (width 0.254) (layer "B.Cu") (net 1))
 (segment (start 79.375 147.955) (end 80.645 146.685) (width 0.254) (layer "B.Cu") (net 1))
 (segment (start 81.915 147.955) (end 104.775 147.955) (width 0.254) (layer "B.Cu") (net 1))
 (segment (start 47.625 69.215) (end 51.435 65.405) (width 0.254) (layer "B.Cu") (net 1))
 (segment (start 80.645 146.685) (end 80.645 144.75) (width 0.254) (layer "B.Cu") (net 1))
 (segment (start 56.515 147.955) (end 79.375 147.955) (width 0.254) (layer "B.Cu") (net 1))
 (segment (start 56.515 147.29) (end 56.515 147.955) (width 0.254) (layer "B.Cu") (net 1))
 (segment (start 107.315 145.415) (end 107.315 144.75) (width 0.254) (layer "B.Cu") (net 1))
 (segment (start 80.645 146.685) (end 81.915 147.955) (width 0.254) (layer "B.Cu") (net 1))
 (segment (start 104.775 147.955) (end 107.315 145.415) (width 0.254) (layer "B.Cu") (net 1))
 (segment (start 79.943971 42.545) (end 80.0608 42.661829) (width 0.254) (layer "F.Cu") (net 16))
 (segment (start 62.495 42.545) (end 79.943971 42.545) (width 0.254) (layer "F.Cu") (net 16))
 (segment (start 79.938518 40.045) (end 80.0608 40.167282) (width 0.254) (layer "F.Cu") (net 15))
 (segment (start 62.865 40.005) (end 63.027282 40.167282) (width 0.254) (layer "F.Cu") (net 15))
 (segment (start 62.495 40.045) (end 79.938518 40.045) (width 0.254) (layer "F.Cu") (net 15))
 (segment (start 62.495 40.045) (end 62.825 40.045) (width 0.254) (layer "F.Cu") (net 15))
 (segment (start 62.825 40.045) (end 62.865 40.005) (width 0.254) (layer "F.Cu") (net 15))
 (segment (start 62.825 40.045) (end 62.865 40.005) (width 0.254) (layer "B.Cu") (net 15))
 (segment (start 62.495 40.045) (end 62.825 40.045) (width 0.254) (layer "B.Cu") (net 15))
 (segment (start 107.315 85.725) (end 108.585 84.455) (width 0.254) (layer "F.Cu") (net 12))
 (segment (start 108.585 84.455) (end 116.205 84.455) (width 0.254) (layer "F.Cu") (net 12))
 (segment (start 107.315 85.06) (end 107.315 85.725) (width 0.254) (layer "F.Cu") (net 12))
 (segment (start 53.975 85.06) (end 63.53 85.06) (width 0.254) (layer "F.Cu") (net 10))
 (segment (start 63.53 85.06) (end 64.135 84.455) (width 0.254) (layer "F.Cu") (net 10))
 (segment (start 53.975 108.585) (end 64.135 108.585) (width 0.254) (layer "F.Cu") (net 52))
 (segment (start 53.975 109.19) (end 53.975 108.585) (width 0.254) (layer "F.Cu") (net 52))
 (segment (start 53.975 134.59) (end 63.53 134.59) (width 0.254) (layer "F.Cu") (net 4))
 (segment (start 63.53 134.59) (end 64.135 133.985) (width 0.254) (layer "F.Cu") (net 4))
 (segment (start 90.2 85.06) (end 90.805 84.455) (width 0.254) (layer "F.Cu") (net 13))
 (segment (start 81.915 85.06) (end 90.2 85.06) (width 0.254) (layer "F.Cu") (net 13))
 (segment (start 80.645 109.19) (end 90.2 109.19) (width 0.254) (layer "F.Cu") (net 19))
 (segment (start 90.2 109.19) (end 90.805 108.585) (width 0.254) (layer "F.Cu") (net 19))
 (segment (start 115.6 134.59) (end 116.205 133.985) (width 0.254) (layer "F.Cu") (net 20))
 (segment (start 107.315 134.59) (end 115.6 134.59) (width 0.254) (layer "F.Cu") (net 20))
 (segment (start 115.6 109.19) (end 116.205 108.585) (width 0.254) (layer "F.Cu") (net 7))
 (segment (start 107.315 109.19) (end 115.6 109.19) (width 0.254) (layer "F.Cu") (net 7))
 (segment (start 80.645 134.59) (end 90.2 134.59) (width 0.254) (layer "F.Cu") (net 2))
 (segment (start 90.2 134.59) (end 90.805 133.985) (width 0.254) (layer "F.Cu") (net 2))
 (segment (start 79.949424 45.045) (end 80.0608 45.156376) (width 0.254) (layer "F.Cu") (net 14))
 (segment (start 62.495 45.045) (end 79.949424 45.045) (width 0.254) (layer "F.Cu") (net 14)))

